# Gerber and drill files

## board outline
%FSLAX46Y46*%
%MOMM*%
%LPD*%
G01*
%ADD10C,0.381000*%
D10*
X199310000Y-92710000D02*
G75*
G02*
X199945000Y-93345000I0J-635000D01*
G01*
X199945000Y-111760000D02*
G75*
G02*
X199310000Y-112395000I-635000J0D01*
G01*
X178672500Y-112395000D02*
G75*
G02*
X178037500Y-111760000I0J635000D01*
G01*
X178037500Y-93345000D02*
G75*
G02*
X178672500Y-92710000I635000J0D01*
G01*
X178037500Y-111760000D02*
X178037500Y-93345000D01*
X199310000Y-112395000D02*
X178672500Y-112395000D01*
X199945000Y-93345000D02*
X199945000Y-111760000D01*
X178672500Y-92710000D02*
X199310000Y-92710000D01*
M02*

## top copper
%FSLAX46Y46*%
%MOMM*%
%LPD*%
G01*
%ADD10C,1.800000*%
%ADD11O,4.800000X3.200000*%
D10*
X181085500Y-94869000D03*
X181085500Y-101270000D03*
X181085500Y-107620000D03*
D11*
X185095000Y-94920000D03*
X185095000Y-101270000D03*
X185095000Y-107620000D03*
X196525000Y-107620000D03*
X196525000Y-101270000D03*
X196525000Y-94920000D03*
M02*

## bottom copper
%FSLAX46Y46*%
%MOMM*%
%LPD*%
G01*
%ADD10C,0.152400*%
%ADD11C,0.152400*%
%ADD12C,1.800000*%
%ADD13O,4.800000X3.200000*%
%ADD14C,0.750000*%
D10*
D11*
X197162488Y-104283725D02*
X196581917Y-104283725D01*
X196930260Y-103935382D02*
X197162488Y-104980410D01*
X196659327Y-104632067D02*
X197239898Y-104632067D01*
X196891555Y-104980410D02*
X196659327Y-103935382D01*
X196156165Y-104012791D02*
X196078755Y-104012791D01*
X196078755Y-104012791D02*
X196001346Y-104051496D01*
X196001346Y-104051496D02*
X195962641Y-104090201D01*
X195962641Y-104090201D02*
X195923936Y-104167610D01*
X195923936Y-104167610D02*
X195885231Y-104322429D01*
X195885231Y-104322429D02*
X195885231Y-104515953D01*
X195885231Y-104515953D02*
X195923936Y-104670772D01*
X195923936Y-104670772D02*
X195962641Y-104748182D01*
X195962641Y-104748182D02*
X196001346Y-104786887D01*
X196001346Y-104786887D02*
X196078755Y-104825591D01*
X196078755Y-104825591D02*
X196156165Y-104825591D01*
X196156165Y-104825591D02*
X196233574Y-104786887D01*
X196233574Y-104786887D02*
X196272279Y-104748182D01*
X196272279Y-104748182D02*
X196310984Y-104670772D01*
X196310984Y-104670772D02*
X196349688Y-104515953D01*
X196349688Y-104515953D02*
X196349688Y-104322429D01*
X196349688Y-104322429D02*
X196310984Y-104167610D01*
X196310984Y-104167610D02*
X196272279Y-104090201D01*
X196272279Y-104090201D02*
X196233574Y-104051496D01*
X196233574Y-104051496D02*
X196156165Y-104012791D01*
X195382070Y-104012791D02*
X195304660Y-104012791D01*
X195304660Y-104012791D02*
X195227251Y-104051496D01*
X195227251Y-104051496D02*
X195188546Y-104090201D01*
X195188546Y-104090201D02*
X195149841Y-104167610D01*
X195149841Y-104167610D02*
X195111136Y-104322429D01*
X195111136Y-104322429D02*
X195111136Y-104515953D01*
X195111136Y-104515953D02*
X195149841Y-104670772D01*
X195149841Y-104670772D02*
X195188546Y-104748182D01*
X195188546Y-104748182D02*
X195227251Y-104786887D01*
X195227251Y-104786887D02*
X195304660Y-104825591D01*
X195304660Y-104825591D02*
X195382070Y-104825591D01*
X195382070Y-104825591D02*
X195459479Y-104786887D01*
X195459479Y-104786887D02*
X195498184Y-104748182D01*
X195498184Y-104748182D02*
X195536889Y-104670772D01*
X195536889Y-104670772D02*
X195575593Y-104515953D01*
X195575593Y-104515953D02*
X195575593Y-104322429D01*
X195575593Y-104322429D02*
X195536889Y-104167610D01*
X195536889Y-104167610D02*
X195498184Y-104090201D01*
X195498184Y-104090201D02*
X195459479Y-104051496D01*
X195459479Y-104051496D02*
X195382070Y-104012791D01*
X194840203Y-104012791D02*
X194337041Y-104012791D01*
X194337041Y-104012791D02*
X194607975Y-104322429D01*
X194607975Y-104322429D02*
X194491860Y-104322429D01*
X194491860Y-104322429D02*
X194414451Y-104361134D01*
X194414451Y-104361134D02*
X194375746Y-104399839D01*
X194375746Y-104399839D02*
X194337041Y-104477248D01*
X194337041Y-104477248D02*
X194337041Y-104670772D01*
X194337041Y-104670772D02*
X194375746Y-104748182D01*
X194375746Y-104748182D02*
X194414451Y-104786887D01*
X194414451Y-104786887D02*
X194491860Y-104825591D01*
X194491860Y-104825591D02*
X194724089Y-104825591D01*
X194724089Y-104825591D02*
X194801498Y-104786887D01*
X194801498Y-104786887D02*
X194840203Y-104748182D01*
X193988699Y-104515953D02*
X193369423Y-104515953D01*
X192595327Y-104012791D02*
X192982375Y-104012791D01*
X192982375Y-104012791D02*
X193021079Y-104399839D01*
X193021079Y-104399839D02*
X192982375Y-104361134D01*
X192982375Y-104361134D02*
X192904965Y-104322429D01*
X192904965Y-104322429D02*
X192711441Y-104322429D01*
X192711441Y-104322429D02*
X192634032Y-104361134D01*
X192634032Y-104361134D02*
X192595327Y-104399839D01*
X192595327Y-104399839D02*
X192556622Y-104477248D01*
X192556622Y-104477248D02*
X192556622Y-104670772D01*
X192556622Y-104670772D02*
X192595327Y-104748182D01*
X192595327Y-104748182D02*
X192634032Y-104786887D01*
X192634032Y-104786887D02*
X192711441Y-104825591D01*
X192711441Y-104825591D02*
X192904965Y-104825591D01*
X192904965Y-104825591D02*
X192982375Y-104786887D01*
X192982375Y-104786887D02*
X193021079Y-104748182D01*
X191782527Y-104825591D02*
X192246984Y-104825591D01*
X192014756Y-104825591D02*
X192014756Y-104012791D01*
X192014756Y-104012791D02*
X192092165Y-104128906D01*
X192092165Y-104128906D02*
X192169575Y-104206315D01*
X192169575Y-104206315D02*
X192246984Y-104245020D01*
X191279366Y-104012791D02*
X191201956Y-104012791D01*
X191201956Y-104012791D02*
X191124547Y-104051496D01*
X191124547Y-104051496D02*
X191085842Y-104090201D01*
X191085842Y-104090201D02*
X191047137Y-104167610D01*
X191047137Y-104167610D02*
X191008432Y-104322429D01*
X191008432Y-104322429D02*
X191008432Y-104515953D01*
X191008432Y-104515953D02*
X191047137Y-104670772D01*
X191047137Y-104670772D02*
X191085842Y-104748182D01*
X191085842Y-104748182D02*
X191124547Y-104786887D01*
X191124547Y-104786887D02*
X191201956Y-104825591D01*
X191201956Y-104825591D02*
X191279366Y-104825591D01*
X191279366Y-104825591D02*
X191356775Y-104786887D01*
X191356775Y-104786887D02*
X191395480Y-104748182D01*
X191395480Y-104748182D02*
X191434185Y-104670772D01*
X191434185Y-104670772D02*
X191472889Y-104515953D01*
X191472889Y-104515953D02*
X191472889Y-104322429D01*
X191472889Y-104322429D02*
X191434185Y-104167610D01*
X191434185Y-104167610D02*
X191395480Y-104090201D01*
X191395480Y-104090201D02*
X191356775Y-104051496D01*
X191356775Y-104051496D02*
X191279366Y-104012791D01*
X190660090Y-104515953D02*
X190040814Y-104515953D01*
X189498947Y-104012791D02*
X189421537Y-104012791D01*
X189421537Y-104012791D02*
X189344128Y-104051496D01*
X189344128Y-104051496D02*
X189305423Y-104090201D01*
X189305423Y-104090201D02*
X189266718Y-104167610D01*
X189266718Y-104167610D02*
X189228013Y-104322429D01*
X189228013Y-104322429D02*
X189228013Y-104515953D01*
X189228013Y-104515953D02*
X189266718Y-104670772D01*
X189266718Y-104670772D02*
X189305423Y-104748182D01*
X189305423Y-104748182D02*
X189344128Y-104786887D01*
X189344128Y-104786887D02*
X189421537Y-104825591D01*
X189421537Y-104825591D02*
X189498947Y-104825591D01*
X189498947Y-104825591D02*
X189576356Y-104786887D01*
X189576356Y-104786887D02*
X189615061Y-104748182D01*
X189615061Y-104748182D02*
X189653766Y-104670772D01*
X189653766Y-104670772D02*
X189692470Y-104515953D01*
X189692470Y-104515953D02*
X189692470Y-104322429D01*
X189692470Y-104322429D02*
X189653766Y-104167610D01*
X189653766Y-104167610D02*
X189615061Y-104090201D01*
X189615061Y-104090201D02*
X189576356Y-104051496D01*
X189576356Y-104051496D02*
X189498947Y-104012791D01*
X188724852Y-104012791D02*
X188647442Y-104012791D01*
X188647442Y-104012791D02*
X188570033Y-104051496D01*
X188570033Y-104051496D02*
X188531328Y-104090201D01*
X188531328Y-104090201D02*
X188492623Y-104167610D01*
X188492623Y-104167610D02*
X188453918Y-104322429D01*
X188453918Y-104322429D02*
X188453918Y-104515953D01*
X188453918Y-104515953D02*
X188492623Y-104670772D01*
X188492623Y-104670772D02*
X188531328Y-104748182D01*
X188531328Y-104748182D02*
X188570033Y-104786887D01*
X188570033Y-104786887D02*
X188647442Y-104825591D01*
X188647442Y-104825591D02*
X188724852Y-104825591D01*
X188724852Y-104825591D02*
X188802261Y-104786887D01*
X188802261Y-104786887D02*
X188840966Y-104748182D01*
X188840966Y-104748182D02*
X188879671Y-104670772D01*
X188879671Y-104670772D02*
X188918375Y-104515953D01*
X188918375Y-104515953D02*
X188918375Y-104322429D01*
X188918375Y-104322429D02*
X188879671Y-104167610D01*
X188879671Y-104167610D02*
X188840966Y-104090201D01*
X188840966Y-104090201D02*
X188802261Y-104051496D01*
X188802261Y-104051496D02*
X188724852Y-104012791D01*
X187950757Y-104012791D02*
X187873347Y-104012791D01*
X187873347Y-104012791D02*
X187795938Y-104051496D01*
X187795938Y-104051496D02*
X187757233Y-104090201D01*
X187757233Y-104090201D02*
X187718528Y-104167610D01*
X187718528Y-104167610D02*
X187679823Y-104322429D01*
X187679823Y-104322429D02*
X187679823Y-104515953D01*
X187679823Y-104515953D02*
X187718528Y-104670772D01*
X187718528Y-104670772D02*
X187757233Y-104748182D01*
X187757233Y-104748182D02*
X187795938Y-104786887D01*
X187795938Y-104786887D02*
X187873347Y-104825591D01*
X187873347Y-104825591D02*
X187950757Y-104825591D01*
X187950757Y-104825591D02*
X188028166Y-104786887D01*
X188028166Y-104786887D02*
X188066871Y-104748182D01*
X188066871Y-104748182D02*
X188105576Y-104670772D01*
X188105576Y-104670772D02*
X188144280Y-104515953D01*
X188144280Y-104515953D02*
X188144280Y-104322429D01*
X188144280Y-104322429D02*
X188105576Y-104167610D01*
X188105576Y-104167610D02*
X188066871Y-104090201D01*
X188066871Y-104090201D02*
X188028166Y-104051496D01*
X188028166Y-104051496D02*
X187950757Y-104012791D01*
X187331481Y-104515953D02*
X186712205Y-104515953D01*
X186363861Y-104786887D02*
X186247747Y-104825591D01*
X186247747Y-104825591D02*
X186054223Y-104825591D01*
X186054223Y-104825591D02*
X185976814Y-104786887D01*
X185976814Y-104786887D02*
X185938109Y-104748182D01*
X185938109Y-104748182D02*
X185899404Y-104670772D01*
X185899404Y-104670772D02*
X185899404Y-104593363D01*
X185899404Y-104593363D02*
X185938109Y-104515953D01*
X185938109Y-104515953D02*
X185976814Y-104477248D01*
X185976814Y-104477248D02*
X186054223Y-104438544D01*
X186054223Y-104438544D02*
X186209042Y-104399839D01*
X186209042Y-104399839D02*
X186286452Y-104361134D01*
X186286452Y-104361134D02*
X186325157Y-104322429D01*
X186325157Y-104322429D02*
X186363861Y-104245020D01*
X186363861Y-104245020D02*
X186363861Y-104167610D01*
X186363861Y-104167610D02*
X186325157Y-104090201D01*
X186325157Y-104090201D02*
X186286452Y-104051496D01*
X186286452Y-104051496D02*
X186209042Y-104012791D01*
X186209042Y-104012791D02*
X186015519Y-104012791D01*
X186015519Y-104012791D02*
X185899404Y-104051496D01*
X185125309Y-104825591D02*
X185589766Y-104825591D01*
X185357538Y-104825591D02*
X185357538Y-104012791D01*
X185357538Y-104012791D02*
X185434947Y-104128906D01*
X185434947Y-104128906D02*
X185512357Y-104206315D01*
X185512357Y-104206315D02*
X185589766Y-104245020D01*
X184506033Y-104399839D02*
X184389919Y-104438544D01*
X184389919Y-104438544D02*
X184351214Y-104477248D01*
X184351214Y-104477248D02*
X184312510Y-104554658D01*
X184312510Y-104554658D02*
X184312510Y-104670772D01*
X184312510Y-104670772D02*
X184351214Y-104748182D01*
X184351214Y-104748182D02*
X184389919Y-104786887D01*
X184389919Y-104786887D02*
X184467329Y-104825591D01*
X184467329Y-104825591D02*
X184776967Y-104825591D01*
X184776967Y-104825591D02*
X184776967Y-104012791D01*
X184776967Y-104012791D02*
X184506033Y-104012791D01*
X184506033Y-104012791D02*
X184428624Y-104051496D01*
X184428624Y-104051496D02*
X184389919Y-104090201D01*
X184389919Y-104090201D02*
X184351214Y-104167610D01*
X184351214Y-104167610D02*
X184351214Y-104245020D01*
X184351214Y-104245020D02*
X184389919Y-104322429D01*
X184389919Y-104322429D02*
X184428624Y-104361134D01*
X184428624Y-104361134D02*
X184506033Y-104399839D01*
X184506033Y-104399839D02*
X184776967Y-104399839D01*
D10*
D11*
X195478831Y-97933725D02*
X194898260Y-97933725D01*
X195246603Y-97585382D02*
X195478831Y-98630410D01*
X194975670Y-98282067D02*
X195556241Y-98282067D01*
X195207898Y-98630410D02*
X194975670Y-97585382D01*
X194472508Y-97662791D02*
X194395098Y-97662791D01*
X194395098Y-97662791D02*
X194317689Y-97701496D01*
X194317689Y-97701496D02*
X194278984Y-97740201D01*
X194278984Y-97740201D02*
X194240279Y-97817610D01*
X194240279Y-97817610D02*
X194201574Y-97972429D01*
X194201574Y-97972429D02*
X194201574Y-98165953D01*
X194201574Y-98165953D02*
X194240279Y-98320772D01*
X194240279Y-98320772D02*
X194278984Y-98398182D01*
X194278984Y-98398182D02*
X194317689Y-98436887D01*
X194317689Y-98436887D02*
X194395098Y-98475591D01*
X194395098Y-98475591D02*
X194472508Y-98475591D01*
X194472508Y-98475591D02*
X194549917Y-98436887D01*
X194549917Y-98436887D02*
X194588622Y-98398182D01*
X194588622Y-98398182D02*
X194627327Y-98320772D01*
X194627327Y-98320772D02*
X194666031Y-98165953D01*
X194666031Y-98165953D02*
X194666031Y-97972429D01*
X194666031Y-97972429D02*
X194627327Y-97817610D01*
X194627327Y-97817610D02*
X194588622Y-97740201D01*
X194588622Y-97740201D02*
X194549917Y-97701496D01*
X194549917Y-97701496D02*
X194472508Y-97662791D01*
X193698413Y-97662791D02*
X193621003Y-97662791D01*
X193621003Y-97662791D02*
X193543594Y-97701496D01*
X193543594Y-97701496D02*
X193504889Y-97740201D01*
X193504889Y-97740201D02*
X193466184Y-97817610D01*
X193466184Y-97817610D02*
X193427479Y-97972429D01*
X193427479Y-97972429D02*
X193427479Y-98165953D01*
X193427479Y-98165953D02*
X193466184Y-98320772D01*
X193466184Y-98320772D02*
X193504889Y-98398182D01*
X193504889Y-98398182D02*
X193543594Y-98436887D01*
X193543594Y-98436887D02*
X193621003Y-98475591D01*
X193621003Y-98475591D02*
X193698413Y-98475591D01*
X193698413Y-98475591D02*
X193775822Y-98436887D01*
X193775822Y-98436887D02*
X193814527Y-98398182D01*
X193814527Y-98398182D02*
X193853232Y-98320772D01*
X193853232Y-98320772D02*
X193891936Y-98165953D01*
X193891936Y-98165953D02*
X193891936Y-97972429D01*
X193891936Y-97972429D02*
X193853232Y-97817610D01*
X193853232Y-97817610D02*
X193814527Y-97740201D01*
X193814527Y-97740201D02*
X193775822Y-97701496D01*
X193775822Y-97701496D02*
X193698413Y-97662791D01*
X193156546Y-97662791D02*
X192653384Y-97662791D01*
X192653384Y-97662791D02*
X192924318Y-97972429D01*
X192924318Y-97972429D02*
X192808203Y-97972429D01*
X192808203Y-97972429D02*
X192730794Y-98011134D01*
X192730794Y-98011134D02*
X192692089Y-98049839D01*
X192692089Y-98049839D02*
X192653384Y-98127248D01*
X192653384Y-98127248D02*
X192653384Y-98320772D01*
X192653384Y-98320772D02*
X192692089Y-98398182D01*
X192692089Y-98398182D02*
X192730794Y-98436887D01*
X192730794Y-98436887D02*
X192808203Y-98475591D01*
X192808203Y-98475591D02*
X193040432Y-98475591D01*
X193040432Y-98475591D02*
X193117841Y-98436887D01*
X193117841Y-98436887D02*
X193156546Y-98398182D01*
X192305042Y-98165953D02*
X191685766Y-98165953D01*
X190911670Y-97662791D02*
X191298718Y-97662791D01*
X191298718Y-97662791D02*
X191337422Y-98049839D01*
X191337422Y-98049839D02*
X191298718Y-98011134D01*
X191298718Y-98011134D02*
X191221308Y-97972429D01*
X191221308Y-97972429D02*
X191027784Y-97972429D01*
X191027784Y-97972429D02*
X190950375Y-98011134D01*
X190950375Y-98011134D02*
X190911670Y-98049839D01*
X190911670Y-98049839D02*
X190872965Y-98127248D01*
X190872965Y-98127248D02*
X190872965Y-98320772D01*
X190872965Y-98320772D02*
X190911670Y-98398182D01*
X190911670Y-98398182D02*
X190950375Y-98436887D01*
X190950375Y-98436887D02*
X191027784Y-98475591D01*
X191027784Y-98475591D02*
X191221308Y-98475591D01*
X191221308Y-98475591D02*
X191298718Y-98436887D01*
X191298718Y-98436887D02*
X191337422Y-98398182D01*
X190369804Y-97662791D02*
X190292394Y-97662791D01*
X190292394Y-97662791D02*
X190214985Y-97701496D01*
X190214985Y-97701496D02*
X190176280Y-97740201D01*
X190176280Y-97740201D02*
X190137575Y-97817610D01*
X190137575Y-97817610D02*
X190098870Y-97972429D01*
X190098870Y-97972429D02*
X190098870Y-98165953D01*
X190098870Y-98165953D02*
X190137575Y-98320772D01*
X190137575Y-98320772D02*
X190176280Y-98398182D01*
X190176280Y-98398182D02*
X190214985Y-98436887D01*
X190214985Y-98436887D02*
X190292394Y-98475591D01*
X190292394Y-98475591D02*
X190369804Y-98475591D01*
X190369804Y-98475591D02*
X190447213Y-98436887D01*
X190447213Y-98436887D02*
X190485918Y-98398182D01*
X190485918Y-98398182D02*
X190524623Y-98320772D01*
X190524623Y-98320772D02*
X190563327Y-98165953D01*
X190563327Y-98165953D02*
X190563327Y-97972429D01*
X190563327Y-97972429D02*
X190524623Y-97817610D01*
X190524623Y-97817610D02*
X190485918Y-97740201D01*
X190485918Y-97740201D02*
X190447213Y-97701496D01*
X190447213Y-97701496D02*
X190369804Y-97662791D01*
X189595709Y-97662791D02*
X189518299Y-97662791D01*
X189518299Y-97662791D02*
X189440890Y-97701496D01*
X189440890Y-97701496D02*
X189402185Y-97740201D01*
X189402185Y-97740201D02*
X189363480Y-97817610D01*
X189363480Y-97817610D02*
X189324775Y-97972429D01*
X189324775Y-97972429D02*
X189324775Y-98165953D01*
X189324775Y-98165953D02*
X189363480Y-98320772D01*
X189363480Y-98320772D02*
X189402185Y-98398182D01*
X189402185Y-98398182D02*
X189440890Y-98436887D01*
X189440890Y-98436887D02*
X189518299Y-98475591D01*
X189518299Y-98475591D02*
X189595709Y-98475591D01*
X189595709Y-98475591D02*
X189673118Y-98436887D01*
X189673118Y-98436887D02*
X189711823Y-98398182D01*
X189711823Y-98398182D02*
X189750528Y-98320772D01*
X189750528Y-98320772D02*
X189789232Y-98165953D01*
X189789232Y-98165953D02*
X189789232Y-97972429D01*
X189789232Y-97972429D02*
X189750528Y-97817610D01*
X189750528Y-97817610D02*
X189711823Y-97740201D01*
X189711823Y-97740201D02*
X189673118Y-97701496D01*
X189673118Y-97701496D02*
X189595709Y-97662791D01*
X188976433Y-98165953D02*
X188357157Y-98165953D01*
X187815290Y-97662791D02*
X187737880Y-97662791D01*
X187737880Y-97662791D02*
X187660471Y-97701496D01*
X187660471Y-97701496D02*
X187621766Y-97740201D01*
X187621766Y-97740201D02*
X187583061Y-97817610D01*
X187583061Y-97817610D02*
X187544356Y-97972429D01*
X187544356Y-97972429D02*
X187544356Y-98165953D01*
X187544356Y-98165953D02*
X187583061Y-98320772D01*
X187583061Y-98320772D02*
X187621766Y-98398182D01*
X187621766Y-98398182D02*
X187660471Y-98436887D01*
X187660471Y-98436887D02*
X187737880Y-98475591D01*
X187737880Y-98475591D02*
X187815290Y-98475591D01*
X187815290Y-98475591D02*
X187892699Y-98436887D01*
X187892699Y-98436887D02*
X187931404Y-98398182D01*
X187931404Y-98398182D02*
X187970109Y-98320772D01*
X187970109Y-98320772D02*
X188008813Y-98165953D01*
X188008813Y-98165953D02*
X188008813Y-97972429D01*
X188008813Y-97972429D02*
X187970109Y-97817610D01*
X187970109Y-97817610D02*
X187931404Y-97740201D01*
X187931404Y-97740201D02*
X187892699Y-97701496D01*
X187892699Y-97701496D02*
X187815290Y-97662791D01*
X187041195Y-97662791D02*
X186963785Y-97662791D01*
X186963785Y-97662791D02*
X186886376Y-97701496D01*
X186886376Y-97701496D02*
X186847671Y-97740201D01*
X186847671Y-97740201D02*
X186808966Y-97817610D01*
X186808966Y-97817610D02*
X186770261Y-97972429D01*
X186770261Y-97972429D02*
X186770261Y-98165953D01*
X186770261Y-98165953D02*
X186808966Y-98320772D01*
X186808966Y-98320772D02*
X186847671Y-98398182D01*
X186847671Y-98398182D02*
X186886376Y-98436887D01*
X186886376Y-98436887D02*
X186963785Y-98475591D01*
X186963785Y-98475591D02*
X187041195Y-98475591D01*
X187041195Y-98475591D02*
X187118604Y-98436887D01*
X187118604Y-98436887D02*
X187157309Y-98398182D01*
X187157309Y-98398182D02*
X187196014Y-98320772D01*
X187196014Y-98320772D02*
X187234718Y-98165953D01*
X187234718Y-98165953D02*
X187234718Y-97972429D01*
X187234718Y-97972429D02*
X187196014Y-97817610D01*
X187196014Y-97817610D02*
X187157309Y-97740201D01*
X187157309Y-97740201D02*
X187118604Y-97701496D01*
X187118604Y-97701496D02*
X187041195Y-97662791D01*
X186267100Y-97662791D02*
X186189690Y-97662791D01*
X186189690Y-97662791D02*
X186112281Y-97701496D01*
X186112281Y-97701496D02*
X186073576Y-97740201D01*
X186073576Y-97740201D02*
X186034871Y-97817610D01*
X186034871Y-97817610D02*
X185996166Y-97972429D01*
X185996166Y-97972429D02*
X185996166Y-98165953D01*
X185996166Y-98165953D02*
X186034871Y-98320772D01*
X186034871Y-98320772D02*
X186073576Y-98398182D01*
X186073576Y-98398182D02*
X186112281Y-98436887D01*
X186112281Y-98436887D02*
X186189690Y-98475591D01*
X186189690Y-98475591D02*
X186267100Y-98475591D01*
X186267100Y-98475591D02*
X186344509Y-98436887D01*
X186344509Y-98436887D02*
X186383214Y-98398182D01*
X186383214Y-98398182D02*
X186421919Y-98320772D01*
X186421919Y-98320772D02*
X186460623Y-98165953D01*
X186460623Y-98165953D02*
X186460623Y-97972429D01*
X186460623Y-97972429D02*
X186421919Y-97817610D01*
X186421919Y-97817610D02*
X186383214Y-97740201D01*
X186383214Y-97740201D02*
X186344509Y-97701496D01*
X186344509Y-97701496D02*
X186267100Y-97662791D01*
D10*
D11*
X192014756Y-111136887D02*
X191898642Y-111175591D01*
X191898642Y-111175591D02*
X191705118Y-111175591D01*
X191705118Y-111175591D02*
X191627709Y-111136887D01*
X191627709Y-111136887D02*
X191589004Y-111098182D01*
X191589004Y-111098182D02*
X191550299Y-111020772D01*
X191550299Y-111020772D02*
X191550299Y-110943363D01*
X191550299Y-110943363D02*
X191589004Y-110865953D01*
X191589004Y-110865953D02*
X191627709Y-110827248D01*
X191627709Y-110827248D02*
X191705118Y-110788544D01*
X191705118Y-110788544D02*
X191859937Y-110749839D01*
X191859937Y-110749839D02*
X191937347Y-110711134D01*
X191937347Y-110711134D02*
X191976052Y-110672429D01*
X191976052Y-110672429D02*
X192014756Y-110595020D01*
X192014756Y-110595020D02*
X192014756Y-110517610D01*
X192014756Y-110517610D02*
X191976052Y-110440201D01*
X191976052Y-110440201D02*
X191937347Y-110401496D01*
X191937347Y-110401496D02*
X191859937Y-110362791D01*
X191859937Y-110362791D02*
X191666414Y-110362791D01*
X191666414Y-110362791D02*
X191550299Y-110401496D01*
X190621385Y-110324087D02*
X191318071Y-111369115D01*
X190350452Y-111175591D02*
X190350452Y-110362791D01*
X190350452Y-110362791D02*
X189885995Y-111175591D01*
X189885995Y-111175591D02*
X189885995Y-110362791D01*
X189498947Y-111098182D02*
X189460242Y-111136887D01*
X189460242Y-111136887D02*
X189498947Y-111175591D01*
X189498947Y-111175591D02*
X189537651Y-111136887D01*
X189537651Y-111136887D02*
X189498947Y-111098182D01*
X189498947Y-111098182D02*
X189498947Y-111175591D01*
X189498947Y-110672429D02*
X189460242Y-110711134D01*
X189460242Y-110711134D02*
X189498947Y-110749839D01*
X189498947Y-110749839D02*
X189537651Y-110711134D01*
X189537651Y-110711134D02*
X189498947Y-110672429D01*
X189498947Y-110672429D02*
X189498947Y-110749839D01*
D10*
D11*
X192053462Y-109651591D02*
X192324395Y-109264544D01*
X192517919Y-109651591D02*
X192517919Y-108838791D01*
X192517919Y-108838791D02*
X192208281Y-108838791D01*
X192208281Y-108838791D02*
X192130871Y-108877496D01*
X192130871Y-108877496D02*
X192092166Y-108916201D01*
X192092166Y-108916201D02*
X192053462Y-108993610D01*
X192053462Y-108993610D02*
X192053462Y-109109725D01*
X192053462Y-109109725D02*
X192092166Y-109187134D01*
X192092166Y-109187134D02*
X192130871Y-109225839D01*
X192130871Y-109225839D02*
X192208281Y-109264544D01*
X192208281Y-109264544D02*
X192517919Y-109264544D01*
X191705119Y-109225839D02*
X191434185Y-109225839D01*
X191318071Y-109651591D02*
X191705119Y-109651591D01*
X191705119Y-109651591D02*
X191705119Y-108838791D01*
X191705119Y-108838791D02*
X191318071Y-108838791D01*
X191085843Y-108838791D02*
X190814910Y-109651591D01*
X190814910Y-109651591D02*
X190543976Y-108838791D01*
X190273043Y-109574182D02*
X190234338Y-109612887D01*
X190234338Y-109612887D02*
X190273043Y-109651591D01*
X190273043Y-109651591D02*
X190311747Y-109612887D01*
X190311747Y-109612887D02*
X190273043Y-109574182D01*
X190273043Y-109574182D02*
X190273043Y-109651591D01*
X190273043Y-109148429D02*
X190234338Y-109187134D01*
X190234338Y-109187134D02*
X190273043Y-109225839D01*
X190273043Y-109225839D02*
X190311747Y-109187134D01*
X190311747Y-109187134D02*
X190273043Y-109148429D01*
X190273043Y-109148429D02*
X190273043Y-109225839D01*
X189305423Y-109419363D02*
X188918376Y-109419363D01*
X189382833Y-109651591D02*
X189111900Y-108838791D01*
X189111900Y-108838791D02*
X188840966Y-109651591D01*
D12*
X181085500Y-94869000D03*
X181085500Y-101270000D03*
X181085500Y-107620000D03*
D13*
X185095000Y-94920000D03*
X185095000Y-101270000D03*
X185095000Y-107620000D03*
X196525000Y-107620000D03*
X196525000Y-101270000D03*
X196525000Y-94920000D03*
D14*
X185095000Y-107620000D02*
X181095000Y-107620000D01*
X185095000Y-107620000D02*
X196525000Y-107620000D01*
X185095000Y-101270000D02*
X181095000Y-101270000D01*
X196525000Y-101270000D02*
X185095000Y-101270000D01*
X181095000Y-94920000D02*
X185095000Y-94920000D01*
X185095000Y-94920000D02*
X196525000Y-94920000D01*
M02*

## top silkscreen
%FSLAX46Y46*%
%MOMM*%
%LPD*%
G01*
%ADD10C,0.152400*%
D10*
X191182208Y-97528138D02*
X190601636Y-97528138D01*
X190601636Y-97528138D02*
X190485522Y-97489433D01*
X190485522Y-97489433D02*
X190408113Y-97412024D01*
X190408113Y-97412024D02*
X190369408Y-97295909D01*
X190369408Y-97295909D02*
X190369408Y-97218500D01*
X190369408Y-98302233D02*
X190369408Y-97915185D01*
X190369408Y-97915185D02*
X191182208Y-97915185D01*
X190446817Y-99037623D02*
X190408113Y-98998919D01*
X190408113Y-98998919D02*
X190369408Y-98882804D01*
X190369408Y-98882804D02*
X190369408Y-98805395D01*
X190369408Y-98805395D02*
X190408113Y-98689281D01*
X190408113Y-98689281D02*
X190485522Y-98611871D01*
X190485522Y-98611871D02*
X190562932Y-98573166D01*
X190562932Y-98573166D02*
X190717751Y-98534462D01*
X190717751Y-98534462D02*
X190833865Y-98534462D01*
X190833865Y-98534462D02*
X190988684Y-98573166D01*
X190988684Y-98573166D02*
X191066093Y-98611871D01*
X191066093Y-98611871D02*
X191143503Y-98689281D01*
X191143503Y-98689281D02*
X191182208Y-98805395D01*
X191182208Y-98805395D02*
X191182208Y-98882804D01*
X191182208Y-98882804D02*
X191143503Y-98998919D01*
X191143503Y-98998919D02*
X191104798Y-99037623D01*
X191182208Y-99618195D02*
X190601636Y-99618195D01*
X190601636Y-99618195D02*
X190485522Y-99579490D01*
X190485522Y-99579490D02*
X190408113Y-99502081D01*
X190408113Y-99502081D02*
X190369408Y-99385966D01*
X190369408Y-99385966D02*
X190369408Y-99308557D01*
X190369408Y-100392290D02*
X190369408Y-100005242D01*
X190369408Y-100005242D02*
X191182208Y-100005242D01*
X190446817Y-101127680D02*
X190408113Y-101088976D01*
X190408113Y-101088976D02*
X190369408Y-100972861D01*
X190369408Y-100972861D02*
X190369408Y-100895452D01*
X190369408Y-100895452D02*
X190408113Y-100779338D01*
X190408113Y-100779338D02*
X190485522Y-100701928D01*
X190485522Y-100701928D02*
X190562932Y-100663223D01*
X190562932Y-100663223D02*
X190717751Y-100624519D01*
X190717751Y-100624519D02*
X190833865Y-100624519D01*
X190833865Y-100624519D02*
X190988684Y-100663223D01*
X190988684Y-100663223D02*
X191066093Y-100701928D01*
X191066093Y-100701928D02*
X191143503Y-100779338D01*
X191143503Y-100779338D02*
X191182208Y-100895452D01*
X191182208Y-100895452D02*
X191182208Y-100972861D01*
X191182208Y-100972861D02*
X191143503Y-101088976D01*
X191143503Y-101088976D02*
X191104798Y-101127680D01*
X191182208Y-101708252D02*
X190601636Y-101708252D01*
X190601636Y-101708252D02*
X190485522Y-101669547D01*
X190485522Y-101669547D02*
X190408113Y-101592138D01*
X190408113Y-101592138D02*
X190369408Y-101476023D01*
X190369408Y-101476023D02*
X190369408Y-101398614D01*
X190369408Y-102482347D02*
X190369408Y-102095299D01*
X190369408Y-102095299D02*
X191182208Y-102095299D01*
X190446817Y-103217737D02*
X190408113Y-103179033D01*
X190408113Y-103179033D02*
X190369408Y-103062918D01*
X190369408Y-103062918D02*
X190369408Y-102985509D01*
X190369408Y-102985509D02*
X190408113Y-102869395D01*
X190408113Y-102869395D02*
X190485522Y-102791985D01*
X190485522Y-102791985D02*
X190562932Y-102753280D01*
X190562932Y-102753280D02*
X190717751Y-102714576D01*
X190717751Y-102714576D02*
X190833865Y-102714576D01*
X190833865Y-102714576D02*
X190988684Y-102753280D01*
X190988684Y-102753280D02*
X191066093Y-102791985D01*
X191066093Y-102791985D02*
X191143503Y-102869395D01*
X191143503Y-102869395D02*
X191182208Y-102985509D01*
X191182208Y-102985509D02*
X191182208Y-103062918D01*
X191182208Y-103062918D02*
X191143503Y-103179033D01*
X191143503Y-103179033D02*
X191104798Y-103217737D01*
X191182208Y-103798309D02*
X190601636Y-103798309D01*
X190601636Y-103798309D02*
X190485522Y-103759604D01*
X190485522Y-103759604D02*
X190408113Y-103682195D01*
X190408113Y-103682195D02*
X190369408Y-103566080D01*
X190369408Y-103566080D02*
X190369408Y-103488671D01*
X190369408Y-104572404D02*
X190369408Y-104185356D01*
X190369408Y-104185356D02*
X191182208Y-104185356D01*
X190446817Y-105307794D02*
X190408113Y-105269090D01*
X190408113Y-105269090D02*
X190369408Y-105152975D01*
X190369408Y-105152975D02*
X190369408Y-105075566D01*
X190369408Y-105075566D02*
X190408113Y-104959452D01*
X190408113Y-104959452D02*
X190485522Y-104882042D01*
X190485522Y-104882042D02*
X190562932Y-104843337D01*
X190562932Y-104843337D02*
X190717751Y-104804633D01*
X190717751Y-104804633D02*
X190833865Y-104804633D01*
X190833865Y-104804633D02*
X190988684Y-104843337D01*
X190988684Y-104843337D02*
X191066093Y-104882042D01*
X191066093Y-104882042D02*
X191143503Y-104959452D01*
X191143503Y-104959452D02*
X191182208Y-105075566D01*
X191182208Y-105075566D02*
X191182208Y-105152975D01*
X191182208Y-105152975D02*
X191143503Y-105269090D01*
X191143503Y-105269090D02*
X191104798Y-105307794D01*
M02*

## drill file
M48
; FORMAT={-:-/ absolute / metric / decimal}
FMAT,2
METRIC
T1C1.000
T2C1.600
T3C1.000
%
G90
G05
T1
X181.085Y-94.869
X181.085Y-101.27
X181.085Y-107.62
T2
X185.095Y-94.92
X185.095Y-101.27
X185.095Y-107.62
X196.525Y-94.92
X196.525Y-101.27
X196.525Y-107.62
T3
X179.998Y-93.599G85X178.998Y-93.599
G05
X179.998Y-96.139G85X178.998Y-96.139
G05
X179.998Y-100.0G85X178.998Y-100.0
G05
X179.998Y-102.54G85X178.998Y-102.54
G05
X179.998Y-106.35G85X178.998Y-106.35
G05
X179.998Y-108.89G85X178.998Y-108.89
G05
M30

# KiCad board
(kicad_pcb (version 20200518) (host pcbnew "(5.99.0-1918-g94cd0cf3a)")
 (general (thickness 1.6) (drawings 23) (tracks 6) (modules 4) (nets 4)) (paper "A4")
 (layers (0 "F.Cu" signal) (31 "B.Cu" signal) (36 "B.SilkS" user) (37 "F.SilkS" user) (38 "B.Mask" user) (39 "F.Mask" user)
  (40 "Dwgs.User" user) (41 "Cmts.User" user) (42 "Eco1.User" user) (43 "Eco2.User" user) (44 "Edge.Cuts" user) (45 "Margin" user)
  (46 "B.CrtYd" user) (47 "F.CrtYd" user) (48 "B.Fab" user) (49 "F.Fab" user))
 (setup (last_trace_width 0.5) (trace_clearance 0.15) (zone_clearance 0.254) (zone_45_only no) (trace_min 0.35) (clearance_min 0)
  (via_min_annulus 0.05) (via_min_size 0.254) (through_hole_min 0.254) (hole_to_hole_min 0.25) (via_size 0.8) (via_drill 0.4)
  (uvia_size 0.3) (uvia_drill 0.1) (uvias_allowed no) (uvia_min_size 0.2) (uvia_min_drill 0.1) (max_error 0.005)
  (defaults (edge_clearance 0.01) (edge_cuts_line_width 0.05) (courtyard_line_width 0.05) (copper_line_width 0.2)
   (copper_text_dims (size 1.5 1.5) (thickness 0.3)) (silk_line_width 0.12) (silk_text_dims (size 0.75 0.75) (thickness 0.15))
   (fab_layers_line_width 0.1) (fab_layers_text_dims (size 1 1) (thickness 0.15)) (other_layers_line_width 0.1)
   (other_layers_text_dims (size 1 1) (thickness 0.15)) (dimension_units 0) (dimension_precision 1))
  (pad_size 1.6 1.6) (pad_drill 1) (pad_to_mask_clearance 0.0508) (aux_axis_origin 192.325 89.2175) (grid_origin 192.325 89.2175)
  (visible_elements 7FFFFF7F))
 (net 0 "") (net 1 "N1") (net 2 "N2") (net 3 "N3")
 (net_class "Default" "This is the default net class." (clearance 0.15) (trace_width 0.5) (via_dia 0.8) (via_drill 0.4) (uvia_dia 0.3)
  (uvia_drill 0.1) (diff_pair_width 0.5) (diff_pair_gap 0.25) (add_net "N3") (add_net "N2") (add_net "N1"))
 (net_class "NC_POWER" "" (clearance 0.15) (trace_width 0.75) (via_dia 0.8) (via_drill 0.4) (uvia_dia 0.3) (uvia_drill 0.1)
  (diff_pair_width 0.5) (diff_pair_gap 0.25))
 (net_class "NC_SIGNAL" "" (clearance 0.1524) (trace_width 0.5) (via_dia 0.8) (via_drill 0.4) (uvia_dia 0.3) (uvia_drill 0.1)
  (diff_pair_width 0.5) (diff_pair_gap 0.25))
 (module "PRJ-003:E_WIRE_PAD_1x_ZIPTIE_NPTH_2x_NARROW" (layer "F.Cu") (at 181.0855 94.869 180)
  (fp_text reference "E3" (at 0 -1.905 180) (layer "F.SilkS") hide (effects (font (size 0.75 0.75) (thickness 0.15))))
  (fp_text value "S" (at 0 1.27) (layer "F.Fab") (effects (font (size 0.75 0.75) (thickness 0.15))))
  (pad "" np_thru_hole oval (at 1.5875 1.27 270) (size 1 2) (drill oval 1 2) (layers *.Cu *.Mask))
  (pad "" np_thru_hole oval (at 1.5875 -1.27 270) (size 1 2) (drill oval 1 2) (layers *.Cu *.Mask))
  (pad "" connect circle (at 0 0 180) (size 1 1) (layers "F.Mask"))
  (pad "1" thru_hole circle (at 0 0 180) (size 1.8 1.8) (drill 1) (layers "B.Cu" "B.Mask") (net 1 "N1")))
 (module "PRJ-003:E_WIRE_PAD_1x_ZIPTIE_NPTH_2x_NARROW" (layer "F.Cu") (at 181.0855 101.27 180)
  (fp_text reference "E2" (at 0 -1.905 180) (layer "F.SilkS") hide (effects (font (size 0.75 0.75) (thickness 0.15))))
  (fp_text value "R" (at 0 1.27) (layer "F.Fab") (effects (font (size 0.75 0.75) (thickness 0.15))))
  (pad "" np_thru_hole oval (at 1.5875 1.27 270) (size 1 2) (drill oval 1 2) (layers *.Cu *.Mask))
  (pad "" np_thru_hole oval (at 1.5875 -1.27 270) (size 1 2) (drill oval 1 2) (layers *.Cu *.Mask))
  (pad "" connect circle (at 0 0 180) (size 1 1) (layers "F.Mask"))
  (pad "1" thru_hole circle (at 0 0 180) (size 1.8 1.8) (drill 1) (layers "B.Cu" "B.Mask") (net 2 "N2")))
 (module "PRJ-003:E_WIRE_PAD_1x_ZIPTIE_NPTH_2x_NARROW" (layer "F.Cu") (at 181.0855 107.62 180)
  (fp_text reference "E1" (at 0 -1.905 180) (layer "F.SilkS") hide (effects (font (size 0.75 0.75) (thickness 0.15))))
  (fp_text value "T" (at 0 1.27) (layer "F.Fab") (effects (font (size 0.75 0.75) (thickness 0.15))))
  (pad "" np_thru_hole oval (at 1.5875 1.27 270) (size 1 2) (drill oval 1 2) (layers *.Cu *.Mask))
  (pad "" np_thru_hole oval (at 1.5875 -1.27 270) (size 1 2) (drill oval 1 2) (layers *.Cu *.Mask))
  (pad "" connect circle (at 0 0 180) (size 1 1) (layers "F.Mask"))
  (pad "1" thru_hole circle (at 0 0 180) (size 1.8 1.8) (drill 1) (layers "B.Cu" "B.Mask") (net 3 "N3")))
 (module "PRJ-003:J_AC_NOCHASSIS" (layer "F.Cu") (at 192.325 90.17)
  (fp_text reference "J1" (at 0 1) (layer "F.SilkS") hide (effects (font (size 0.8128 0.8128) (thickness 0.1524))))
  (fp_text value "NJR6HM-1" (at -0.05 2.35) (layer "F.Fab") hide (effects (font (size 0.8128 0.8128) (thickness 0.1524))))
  (pad "" connect circle (at 4.2 4.75) (size 1.6 1.6) (layers "F.Mask"))
  (pad "" connect circle (at 4.2 11.1) (size 1.6 1.6) (layers "F.Mask"))
  (pad "" connect circle (at 4.2 17.45) (size 1.6 1.6) (layers "F.Mask"))
  (pad "" connect circle (at -7.23 17.45) (size 1.6 1.6) (layers "F.Mask"))
  (pad "" connect circle (at -7.23 11.1) (size 1.6 1.6) (layers "F.Mask"))
  (pad "" connect circle (at -7.23 4.75) (size 1.6 1.6) (layers "F.Mask"))
  (pad "S" thru_hole oval (at -7.23 4.75) (size 4.8 3.2) (drill 1.6) (layers "B.Cu" "B.Mask") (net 1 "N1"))
  (pad "R" thru_hole oval (at -7.23 11.1) (size 4.8 3.2) (drill 1.6) (layers "B.Cu" "B.Mask") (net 2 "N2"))
  (pad "T" thru_hole oval (at -7.23 17.45) (size 4.8 3.2) (drill 1.6) (layers "B.Cu" "B.Mask") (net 3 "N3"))
  (pad "TN" thru_hole oval (at 4.2 17.45) (size 4.8 3.2) (drill 1.6) (layers "B.Cu" "B.Mask") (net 3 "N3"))
  (pad "RN" thru_hole oval (at 4.2 11.1) (size 4.8 3.2) (drill 1.6) (layers "B.Cu" "B.Mask") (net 2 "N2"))
  (pad "SN" thru_hole oval (at 4.2 4.75) (size 4.8 3.2) (drill 1.6) (layers "B.Cu" "B.Mask") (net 1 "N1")))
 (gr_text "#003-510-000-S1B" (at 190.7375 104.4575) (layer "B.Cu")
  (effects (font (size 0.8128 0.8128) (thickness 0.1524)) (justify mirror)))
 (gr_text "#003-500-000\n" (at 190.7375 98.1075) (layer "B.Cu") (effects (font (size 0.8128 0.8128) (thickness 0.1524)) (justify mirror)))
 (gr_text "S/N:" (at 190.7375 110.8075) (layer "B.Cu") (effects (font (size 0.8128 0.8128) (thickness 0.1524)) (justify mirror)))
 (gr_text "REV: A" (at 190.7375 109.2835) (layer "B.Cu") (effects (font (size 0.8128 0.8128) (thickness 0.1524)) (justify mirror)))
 (gr_arc (start 199.31 93.345) (end 199.945 93.345) (angle -90) (layer "Edge.Cuts") (width 0.381))
 (gr_arc (start 199.31 111.76) (end 199.31 112.395) (angle -90) (layer "Edge.Cuts") (width 0.381))
 (gr_arc (start 178.6725 111.76) (end 178.0375 111.76) (angle -90) (layer "Edge.Cuts") (width 0.381))
 (gr_arc (start 178.6725 93.345) (end 178.6725 92.71) (angle -90) (layer "Edge.Cuts") (width 0.381))
 (gr_line (start 178.0375 111.76) (end 178.0375 93.345) (layer "Edge.Cuts") (width 0.381))
 (gr_line (start 199.31 112.395) (end 178.6725 112.395) (layer "Edge.Cuts") (width 0.381))
 (gr_line (start 199.945 93.345) (end 199.945 111.76) (layer "Edge.Cuts") (width 0.381))
 (gr_line (start 178.6725 92.71) (end 199.31 92.71) (layer "Edge.Cuts") (width 0.381))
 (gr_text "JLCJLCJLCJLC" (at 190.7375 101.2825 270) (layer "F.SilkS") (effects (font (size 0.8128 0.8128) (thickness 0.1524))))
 (segment (start 185.095 107.62) (end 181.095 107.62) (width 0.75) (layer "B.Cu") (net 3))
 (segment (start 185.095 107.62) (end 196.525 107.62) (width 0.75) (layer "B.Cu") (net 3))
 (segment (start 185.095 101.27) (end 181.095 101.27) (width 0.75) (layer "B.Cu") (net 2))
 (segment (start 196.525 101.27) (end 185.095 101.27) (width 0.75) (layer "B.Cu") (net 2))
 (segment (start 181.095 94.92) (end 185.095 94.92) (width 0.75) (layer "B.Cu") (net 1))
 (segment (start 185.095 94.92) (end 196.525 94.92) (width 0.75) (layer "B.Cu") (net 1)))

